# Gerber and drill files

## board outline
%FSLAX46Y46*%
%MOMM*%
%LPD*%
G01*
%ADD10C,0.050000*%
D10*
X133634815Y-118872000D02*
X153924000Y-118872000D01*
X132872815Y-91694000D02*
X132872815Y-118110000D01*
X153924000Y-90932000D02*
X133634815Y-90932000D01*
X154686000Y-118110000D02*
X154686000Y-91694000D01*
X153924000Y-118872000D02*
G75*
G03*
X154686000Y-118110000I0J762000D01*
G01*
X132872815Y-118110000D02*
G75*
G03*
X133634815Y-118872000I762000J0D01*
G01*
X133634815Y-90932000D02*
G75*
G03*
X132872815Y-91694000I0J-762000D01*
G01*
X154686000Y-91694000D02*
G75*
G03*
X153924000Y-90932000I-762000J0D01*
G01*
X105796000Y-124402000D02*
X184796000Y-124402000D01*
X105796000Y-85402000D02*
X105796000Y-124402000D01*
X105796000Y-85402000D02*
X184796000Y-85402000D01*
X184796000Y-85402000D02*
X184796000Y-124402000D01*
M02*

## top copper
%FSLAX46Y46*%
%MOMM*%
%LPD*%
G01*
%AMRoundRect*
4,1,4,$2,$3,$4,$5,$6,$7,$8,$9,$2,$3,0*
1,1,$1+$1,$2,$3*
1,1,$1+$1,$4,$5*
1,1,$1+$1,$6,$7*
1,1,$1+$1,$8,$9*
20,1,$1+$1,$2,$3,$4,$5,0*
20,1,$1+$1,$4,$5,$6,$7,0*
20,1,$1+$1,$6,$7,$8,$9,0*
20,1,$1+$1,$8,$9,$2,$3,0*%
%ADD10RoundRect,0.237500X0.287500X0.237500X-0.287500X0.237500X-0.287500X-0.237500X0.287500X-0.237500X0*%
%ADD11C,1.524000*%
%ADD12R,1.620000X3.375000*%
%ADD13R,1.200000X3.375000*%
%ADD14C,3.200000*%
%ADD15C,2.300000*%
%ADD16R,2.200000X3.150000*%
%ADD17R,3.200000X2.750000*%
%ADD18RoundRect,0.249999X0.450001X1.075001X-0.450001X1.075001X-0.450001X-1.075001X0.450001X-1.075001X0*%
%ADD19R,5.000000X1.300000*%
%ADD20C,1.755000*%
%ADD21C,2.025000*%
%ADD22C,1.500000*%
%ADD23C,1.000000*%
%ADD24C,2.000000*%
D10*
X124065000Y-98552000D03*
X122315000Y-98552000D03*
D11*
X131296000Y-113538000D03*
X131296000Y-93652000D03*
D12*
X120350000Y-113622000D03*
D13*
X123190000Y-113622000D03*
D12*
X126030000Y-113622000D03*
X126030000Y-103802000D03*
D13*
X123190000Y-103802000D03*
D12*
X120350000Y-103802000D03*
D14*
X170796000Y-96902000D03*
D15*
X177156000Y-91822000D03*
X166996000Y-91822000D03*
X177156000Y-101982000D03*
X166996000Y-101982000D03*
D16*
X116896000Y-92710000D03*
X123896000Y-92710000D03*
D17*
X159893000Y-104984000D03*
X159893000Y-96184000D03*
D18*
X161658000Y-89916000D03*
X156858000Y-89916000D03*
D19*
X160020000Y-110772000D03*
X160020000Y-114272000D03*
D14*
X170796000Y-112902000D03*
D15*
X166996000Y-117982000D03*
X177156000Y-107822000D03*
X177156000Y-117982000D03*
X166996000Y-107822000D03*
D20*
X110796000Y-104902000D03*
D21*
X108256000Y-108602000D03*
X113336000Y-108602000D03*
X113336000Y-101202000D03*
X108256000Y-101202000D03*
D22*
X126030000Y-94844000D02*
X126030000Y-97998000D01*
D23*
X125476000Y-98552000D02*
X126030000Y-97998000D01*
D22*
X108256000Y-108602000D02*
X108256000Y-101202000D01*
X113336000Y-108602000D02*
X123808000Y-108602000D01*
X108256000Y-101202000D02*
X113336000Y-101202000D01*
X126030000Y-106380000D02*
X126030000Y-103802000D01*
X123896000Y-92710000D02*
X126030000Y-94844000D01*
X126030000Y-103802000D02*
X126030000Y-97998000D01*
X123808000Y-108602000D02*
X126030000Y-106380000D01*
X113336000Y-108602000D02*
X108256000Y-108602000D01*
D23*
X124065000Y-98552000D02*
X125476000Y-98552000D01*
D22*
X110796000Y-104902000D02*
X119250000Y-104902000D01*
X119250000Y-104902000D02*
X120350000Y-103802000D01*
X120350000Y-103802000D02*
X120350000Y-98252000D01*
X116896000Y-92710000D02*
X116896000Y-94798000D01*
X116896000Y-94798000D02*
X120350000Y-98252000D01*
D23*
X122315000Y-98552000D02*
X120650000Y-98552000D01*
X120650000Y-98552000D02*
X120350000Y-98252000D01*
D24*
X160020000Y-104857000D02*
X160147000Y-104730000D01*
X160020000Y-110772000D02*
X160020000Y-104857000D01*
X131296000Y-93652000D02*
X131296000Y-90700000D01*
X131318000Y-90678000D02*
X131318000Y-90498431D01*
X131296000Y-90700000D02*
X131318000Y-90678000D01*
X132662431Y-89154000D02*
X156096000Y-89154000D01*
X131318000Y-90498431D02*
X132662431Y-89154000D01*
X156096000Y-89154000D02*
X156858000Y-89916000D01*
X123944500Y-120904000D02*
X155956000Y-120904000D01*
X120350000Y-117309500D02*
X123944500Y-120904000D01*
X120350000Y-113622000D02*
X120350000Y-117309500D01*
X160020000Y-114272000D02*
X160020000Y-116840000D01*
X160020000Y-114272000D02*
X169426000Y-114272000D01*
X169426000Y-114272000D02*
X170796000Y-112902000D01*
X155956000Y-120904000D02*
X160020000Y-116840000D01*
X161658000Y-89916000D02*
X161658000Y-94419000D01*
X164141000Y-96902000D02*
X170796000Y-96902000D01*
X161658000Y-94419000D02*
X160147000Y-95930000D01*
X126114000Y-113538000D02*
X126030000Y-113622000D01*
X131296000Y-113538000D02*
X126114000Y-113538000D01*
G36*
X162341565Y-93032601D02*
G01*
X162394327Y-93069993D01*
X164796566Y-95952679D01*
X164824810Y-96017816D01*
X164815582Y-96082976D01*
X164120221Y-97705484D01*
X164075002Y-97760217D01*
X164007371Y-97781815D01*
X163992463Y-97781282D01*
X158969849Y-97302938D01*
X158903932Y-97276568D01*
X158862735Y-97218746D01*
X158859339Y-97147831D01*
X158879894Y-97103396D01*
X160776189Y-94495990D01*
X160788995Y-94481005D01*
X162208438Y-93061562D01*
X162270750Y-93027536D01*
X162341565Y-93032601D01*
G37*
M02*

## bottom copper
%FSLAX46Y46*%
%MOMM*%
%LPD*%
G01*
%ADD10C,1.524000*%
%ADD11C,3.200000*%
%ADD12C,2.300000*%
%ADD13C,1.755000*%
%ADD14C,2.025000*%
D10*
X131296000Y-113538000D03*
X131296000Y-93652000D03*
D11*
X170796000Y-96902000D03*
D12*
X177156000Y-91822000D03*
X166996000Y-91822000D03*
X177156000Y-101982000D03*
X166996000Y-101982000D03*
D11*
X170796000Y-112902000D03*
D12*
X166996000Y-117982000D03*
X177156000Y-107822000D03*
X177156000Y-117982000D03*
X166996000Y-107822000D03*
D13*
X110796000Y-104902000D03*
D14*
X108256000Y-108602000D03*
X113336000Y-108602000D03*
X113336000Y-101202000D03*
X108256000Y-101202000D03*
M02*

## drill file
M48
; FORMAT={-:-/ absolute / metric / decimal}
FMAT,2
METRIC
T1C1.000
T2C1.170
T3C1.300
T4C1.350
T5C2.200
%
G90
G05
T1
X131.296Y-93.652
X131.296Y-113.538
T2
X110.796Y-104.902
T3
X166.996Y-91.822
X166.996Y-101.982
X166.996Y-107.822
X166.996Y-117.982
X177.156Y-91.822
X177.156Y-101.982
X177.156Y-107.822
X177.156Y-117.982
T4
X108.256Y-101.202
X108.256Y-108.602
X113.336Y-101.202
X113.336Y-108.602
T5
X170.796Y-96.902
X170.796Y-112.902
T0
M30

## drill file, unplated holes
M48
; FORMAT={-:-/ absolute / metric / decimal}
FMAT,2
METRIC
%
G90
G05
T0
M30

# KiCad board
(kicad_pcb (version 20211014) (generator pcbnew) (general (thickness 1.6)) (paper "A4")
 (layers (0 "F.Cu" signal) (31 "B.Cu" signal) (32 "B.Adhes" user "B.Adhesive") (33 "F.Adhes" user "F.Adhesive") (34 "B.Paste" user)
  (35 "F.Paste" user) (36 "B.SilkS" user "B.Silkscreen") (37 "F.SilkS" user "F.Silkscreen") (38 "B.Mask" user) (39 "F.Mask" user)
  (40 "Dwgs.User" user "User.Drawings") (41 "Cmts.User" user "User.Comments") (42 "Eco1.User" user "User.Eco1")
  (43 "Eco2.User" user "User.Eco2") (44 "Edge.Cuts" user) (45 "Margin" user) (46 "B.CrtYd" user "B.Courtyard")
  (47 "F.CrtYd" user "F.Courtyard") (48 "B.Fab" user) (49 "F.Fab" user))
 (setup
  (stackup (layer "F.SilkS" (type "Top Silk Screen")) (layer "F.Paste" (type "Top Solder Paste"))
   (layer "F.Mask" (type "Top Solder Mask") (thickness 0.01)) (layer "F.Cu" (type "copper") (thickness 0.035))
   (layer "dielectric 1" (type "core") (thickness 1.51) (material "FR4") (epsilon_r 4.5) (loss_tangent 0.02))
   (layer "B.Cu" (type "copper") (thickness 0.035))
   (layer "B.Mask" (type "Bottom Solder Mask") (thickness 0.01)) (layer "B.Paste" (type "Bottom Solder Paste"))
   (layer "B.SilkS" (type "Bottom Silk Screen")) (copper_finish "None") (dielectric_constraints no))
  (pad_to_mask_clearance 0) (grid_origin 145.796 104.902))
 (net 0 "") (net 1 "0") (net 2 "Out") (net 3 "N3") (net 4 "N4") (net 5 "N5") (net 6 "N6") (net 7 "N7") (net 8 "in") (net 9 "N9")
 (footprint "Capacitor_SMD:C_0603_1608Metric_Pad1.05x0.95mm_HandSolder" (layer "F.Cu") (at 123.19 98.552 180)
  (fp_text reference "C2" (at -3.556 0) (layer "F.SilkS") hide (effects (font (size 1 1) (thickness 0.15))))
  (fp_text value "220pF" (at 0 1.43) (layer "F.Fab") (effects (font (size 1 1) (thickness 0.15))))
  (pad "1" smd roundrect locked (at -0.875 0 180) (size 1.05 0.95) (layers "F.Cu" "F.Paste" "F.Mask") (roundrect_rratio 0.25) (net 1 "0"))
  (pad "2" smd roundrect locked (at 0.875 0 180) (size 1.05 0.95) (layers "F.Cu" "F.Paste" "F.Mask") (roundrect_rratio 0.25) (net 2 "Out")))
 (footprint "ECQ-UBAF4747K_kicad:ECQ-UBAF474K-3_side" (layer "F.Cu") (at 133.296 104.902 180)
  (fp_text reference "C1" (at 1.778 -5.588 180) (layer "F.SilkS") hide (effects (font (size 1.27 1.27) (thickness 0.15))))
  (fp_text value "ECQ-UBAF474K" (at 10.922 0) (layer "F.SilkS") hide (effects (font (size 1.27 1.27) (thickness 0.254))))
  (pad "1" thru_hole circle (at 2 11.25 180) (size 1.524 1.524) (drill 1) (layers *.Cu *.Mask) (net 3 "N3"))
  (pad "2" thru_hole circle (at 2 -8.636 180) (size 1.524 1.524) (drill 1) (layers *.Cu *.Mask) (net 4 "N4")))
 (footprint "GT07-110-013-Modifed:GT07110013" (layer "F.Cu") (at 123.19 108.712 180)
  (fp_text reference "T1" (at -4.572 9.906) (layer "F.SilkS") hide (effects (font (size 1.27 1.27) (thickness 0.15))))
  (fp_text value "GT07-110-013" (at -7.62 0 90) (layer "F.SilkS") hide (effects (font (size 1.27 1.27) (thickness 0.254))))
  (pad "1" smd rect (at 2.84 -4.91 180) (size 1.62 3.375) (layers "F.Cu" "F.Paste" "F.Mask") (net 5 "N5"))
  (pad "2" smd rect (at 0 -4.91 180) (size 1.2 3.375) (layers "F.Cu" "F.Paste" "F.Mask") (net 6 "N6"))
  (pad "3" smd rect (at -2.84 -4.91 180) (size 1.62 3.375) (layers "F.Cu" "F.Paste" "F.Mask") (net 4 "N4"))
  (pad "4" smd rect (at -2.84 4.91 180) (size 1.62 3.375) (layers "F.Cu" "F.Paste" "F.Mask") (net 1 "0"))
  (pad "5" smd rect (at 0 4.91 180) (size 1.2 3.375) (layers "F.Cu" "F.Paste" "F.Mask") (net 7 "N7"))
  (pad "6" smd rect (at 2.84 4.91 180) (size 1.62 3.375) (layers "F.Cu" "F.Paste" "F.Mask") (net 2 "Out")))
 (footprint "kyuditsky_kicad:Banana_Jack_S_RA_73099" (layer "F.Cu") (at 170.796 96.902)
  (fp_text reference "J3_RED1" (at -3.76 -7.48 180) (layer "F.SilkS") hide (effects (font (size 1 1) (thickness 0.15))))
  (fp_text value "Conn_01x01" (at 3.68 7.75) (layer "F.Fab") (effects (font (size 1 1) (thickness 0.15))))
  (pad "1" thru_hole circle (at 0 0) (size 3.2 3.2) (drill 2.2) (layers *.Cu *.Mask) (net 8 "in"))
  (pad "2" thru_hole circle locked (at 6.36 -5.08) (size 2.3 2.3) (drill 1.3) (layers *.Cu *.Mask))
  (pad "2" thru_hole circle locked (at -3.8 -5.08) (size 2.3 2.3) (drill 1.3) (layers *.Cu *.Mask))
  (pad "2" thru_hole circle locked (at 6.36 5.08) (size 2.3 2.3) (drill 1.3) (layers *.Cu *.Mask))
  (pad "2" thru_hole circle locked (at -3.8 5.08) (size 2.3 2.3) (drill 1.3) (layers *.Cu *.Mask)))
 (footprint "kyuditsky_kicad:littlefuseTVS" (layer "F.Cu") (at 120.396 92.71)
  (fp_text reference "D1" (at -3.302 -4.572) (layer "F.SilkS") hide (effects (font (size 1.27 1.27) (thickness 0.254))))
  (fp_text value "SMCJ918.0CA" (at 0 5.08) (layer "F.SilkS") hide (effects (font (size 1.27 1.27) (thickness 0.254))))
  (pad "1" smd rect locked (at -3.5 0) (size 2.2 3.15) (layers "F.Cu" "F.Paste" "F.Mask") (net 2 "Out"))
  (pad "2" smd rect locked (at 3.5 0) (size 2.2 3.15) (layers "F.Cu" "F.Paste" "F.Mask") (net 1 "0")))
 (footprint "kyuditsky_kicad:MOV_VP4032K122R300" (layer "F.Cu") (at 159.766 100.584 90)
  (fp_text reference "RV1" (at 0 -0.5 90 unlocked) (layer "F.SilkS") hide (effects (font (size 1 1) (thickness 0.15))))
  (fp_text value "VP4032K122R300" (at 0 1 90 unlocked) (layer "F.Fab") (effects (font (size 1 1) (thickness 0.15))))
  (pad "1" smd rect (at -4.4 0.127 90) (size 2.75 3.2) (layers "F.Cu" "F.Paste" "F.Mask") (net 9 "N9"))
  (pad "2" smd rect (at 4.4 0.127 90) (size 2.75 3.2) (layers "F.Cu" "F.Paste" "F.Mask") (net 8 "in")))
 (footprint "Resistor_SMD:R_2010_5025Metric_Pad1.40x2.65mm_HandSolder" (layer "F.Cu") (at 159.258 89.916 180)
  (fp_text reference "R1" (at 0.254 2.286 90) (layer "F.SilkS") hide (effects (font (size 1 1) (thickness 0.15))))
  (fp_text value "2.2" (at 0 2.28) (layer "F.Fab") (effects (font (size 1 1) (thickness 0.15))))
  (pad "1" smd roundrect (at -2.4 0 180) (size 1.4 2.65) (layers "F.Cu" "F.Paste" "F.Mask") (roundrect_rratio 0.1785707143) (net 8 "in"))
  (pad "2" smd roundrect (at 2.4 0 180) (size 1.4 2.65) (layers "F.Cu" "F.Paste" "F.Mask") (roundrect_rratio 0.1785707143) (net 3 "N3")))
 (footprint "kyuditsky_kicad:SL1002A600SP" (layer "F.Cu") (at 160.02 112.522 -90)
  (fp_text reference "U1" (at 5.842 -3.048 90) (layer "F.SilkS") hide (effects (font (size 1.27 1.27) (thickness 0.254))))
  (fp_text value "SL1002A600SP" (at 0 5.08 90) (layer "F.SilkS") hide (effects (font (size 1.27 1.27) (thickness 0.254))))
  (pad "1" smd rect locked (at -1.75 0 270) (size 1.3 5) (layers "F.Cu" "F.Paste" "F.Mask") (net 9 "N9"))
  (pad "2" smd rect locked (at 1.75 0 270) (size 1.3 5) (layers "F.Cu" "F.Paste" "F.Mask") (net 5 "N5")))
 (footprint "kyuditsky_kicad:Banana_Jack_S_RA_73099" (layer "F.Cu") (at 170.796 112.902)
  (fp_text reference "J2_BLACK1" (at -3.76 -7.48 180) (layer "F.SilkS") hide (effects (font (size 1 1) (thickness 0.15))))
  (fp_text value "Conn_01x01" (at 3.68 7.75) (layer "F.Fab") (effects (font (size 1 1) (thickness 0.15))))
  (pad "1" thru_hole circle locked (at 0 0) (size 3.2 3.2) (drill 2.2) (layers *.Cu *.Mask) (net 5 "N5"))
  (pad "2" thru_hole circle locked (at -3.8 5.08) (size 2.3 2.3) (drill 1.3) (layers *.Cu *.Mask))
  (pad "2" thru_hole circle locked (at 6.36 -5.08) (size 2.3 2.3) (drill 1.3) (layers *.Cu *.Mask))
  (pad "2" thru_hole circle locked (at 6.36 5.08) (size 2.3 2.3) (drill 1.3) (layers *.Cu *.Mask))
  (pad "2" thru_hole circle locked (at -3.8 -5.08) (size 2.3 2.3) (drill 1.3) (layers *.Cu *.Mask)))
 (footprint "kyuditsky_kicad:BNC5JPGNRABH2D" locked (layer "F.Cu") (at 110.796 104.902 90)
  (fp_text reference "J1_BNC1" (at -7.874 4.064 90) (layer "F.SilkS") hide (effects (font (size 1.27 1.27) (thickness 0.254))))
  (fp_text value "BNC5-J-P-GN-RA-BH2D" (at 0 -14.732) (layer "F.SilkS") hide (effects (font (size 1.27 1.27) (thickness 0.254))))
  (pad "1" thru_hole circle locked (at 0 0 90) (size 1.755 1.755) (drill 1.17) (layers *.Cu *.Mask) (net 2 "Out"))
  (pad "2" thru_hole circle locked (at -3.7 -2.54 90) (size 2.025 2.025) (drill 1.35) (layers *.Cu *.Mask) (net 1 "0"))
  (pad "3" thru_hole circle locked (at -3.7 2.54 90) (size 2.025 2.025) (drill 1.35) (layers *.Cu *.Mask) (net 1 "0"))
  (pad "4" thru_hole circle locked (at 3.7 2.54 90) (size 2.025 2.025) (drill 1.35) (layers *.Cu *.Mask) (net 1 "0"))
  (pad "5" thru_hole circle locked (at 3.7 -2.54 90) (size 2.025 2.025) (drill 1.35) (layers *.Cu *.Mask) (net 1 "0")))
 (gr_line (start 105.796 124.402) (end 184.796 124.402) (layer "Edge.Cuts") (width 0.05))
 (gr_arc (start 153.924 90.932) (mid 154.462815 91.155185) (end 154.686 91.694) (layer "Edge.Cuts") (width 0.05))
 (gr_line (start 132.872815 91.694) (end 132.872815 118.11) (layer "Edge.Cuts") (width 0.05))
 (gr_line (start 105.796 85.402) (end 105.796 124.402) (layer "Edge.Cuts") (width 0.05))
 (gr_line (start 105.796 85.402) (end 184.796 85.402) (layer "Edge.Cuts") (width 0.05))
 (gr_arc (start 133.634815 118.872) (mid 133.096 118.648815) (end 132.872815 118.11) (layer "Edge.Cuts") (width 0.05))
 (gr_line (start 133.634815 118.872) (end 153.924 118.872) (layer "Edge.Cuts") (width 0.05))
 (gr_line (start 153.924 90.932) (end 133.634815 90.932) (layer "Edge.Cuts") (width 0.05))
 (gr_line (start 154.686 118.11) (end 154.686 91.694) (layer "Edge.Cuts") (width 0.05))
 (gr_arc (start 132.872815 91.694) (mid 133.096 91.155185) (end 133.634815 90.932) (layer "Edge.Cuts") (width 0.05))
 (gr_arc (start 154.686 118.11) (mid 154.462815 118.648815) (end 153.924 118.872) (layer "Edge.Cuts") (width 0.05))
 (gr_line (start 184.796 85.402) (end 184.796 124.402) (layer "Edge.Cuts") (width 0.05))
 (segment (start 126.03 94.844) (end 126.03 97.998) (width 1.5) (layer "F.Cu") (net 1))
 (segment (start 125.476 98.552) (end 126.03 97.998) (width 1) (layer "F.Cu") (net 1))
 (segment (start 108.256 108.602) (end 108.256 101.202) (width 1.5) (layer "F.Cu") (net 1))
 (segment (start 113.336 108.602) (end 123.808 108.602) (width 1.5) (layer "F.Cu") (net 1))
 (segment (start 108.256 101.202) (end 113.336 101.202) (width 1.5) (layer "F.Cu") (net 1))
 (segment (start 126.03 106.38) (end 126.03 103.802) (width 1.5) (layer "F.Cu") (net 1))
 (segment (start 123.896 92.71) (end 126.03 94.844) (width 1.5) (layer "F.Cu") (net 1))
 (segment (start 126.03 103.802) (end 126.03 97.998) (width 1.5) (layer "F.Cu") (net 1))
 (segment (start 123.808 108.602) (end 126.03 106.38) (width 1.5) (layer "F.Cu") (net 1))
 (segment (start 113.336 108.602) (end 108.256 108.602) (width 1.5) (layer "F.Cu") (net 1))
 (segment (start 124.065 98.552) (end 125.476 98.552) (width 1) (layer "F.Cu") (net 1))
 (segment (start 110.796 104.902) (end 119.25 104.902) (width 1.5) (layer "F.Cu") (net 2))
 (segment (start 119.25 104.902) (end 120.35 103.802) (width 1.5) (layer "F.Cu") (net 2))
 (segment (start 120.35 103.802) (end 120.35 98.252) (width 1.5) (layer "F.Cu") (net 2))
 (segment (start 116.896 92.71) (end 116.896 94.798) (width 1.5) (layer "F.Cu") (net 2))
 (segment (start 116.896 94.798) (end 120.35 98.252) (width 1.5) (layer "F.Cu") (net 2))
 (segment (start 122.315 98.552) (end 120.65 98.552) (width 1) (layer "F.Cu") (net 2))
 (segment (start 120.65 98.552) (end 120.35 98.252) (width 1) (layer "F.Cu") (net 2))
 (segment (start 160.02 104.857) (end 160.147 104.73) (width 2) (layer "F.Cu") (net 9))
 (segment (start 160.02 110.772) (end 160.02 104.857) (width 2) (layer "F.Cu") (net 9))
 (segment (start 131.296 93.652) (end 131.296 90.7) (width 2) (layer "F.Cu") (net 3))
 (segment (start 131.318 90.678) (end 131.318 90.498431) (width 2) (layer "F.Cu") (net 3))
 (segment (start 131.296 90.7) (end 131.318 90.678) (width 2) (layer "F.Cu") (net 3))
 (segment (start 132.662431 89.154) (end 156.096 89.154) (width 2) (layer "F.Cu") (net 3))
 (segment (start 131.318 90.498431) (end 132.662431 89.154) (width 2) (layer "F.Cu") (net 3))
 (segment (start 156.096 89.154) (end 156.858 89.916) (width 2) (layer "F.Cu") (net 3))
 (segment (start 123.9445 120.904) (end 155.956 120.904) (width 2) (layer "F.Cu") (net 5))
 (segment (start 120.35 117.3095) (end 123.9445 120.904) (width 2) (layer "F.Cu") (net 5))
 (segment (start 120.35 113.622) (end 120.35 117.3095) (width 2) (layer "F.Cu") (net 5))
 (segment (start 160.02 114.272) (end 160.02 116.84) (width 2) (layer "F.Cu") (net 5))
 (segment (start 160.02 114.272) (end 169.426 114.272) (width 2) (layer "F.Cu") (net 5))
 (segment (start 169.426 114.272) (end 170.796 112.902) (width 2) (layer "F.Cu") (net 5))
 (segment (start 155.956 120.904) (end 160.02 116.84) (width 2) (layer "F.Cu") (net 5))
 (segment (start 126.114 113.538) (end 126.03 113.622) (width 2) (layer "F.Cu") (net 4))
 (segment (start 131.296 113.538) (end 126.114 113.538) (width 2) (layer "F.Cu") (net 4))
 (segment (start 161.658 89.916) (end 161.658 94.419) (width 2) (layer "F.Cu") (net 8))
 (segment (start 164.141 96.902) (end 170.796 96.902) (width 2) (layer "F.Cu") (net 8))
 (segment (start 161.658 94.419) (end 160.147 95.93) (width 2) (layer "F.Cu") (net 8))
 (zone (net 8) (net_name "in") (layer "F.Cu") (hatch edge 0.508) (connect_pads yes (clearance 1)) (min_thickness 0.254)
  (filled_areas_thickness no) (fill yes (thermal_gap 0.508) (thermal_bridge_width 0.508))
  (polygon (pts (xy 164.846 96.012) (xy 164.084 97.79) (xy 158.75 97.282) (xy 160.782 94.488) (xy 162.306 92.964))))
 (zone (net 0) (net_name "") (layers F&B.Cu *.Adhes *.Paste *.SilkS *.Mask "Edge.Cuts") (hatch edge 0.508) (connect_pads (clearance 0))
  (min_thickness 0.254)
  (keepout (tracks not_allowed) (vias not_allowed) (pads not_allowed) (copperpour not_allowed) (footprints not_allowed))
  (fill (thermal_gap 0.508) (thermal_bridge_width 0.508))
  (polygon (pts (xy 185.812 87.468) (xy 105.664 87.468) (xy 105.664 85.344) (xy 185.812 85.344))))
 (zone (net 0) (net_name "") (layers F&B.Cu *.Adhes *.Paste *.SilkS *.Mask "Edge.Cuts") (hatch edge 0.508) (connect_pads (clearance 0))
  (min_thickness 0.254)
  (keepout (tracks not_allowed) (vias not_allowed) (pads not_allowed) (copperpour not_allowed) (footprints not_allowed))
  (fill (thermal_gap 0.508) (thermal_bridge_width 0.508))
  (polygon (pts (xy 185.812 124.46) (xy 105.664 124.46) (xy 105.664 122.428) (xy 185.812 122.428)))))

